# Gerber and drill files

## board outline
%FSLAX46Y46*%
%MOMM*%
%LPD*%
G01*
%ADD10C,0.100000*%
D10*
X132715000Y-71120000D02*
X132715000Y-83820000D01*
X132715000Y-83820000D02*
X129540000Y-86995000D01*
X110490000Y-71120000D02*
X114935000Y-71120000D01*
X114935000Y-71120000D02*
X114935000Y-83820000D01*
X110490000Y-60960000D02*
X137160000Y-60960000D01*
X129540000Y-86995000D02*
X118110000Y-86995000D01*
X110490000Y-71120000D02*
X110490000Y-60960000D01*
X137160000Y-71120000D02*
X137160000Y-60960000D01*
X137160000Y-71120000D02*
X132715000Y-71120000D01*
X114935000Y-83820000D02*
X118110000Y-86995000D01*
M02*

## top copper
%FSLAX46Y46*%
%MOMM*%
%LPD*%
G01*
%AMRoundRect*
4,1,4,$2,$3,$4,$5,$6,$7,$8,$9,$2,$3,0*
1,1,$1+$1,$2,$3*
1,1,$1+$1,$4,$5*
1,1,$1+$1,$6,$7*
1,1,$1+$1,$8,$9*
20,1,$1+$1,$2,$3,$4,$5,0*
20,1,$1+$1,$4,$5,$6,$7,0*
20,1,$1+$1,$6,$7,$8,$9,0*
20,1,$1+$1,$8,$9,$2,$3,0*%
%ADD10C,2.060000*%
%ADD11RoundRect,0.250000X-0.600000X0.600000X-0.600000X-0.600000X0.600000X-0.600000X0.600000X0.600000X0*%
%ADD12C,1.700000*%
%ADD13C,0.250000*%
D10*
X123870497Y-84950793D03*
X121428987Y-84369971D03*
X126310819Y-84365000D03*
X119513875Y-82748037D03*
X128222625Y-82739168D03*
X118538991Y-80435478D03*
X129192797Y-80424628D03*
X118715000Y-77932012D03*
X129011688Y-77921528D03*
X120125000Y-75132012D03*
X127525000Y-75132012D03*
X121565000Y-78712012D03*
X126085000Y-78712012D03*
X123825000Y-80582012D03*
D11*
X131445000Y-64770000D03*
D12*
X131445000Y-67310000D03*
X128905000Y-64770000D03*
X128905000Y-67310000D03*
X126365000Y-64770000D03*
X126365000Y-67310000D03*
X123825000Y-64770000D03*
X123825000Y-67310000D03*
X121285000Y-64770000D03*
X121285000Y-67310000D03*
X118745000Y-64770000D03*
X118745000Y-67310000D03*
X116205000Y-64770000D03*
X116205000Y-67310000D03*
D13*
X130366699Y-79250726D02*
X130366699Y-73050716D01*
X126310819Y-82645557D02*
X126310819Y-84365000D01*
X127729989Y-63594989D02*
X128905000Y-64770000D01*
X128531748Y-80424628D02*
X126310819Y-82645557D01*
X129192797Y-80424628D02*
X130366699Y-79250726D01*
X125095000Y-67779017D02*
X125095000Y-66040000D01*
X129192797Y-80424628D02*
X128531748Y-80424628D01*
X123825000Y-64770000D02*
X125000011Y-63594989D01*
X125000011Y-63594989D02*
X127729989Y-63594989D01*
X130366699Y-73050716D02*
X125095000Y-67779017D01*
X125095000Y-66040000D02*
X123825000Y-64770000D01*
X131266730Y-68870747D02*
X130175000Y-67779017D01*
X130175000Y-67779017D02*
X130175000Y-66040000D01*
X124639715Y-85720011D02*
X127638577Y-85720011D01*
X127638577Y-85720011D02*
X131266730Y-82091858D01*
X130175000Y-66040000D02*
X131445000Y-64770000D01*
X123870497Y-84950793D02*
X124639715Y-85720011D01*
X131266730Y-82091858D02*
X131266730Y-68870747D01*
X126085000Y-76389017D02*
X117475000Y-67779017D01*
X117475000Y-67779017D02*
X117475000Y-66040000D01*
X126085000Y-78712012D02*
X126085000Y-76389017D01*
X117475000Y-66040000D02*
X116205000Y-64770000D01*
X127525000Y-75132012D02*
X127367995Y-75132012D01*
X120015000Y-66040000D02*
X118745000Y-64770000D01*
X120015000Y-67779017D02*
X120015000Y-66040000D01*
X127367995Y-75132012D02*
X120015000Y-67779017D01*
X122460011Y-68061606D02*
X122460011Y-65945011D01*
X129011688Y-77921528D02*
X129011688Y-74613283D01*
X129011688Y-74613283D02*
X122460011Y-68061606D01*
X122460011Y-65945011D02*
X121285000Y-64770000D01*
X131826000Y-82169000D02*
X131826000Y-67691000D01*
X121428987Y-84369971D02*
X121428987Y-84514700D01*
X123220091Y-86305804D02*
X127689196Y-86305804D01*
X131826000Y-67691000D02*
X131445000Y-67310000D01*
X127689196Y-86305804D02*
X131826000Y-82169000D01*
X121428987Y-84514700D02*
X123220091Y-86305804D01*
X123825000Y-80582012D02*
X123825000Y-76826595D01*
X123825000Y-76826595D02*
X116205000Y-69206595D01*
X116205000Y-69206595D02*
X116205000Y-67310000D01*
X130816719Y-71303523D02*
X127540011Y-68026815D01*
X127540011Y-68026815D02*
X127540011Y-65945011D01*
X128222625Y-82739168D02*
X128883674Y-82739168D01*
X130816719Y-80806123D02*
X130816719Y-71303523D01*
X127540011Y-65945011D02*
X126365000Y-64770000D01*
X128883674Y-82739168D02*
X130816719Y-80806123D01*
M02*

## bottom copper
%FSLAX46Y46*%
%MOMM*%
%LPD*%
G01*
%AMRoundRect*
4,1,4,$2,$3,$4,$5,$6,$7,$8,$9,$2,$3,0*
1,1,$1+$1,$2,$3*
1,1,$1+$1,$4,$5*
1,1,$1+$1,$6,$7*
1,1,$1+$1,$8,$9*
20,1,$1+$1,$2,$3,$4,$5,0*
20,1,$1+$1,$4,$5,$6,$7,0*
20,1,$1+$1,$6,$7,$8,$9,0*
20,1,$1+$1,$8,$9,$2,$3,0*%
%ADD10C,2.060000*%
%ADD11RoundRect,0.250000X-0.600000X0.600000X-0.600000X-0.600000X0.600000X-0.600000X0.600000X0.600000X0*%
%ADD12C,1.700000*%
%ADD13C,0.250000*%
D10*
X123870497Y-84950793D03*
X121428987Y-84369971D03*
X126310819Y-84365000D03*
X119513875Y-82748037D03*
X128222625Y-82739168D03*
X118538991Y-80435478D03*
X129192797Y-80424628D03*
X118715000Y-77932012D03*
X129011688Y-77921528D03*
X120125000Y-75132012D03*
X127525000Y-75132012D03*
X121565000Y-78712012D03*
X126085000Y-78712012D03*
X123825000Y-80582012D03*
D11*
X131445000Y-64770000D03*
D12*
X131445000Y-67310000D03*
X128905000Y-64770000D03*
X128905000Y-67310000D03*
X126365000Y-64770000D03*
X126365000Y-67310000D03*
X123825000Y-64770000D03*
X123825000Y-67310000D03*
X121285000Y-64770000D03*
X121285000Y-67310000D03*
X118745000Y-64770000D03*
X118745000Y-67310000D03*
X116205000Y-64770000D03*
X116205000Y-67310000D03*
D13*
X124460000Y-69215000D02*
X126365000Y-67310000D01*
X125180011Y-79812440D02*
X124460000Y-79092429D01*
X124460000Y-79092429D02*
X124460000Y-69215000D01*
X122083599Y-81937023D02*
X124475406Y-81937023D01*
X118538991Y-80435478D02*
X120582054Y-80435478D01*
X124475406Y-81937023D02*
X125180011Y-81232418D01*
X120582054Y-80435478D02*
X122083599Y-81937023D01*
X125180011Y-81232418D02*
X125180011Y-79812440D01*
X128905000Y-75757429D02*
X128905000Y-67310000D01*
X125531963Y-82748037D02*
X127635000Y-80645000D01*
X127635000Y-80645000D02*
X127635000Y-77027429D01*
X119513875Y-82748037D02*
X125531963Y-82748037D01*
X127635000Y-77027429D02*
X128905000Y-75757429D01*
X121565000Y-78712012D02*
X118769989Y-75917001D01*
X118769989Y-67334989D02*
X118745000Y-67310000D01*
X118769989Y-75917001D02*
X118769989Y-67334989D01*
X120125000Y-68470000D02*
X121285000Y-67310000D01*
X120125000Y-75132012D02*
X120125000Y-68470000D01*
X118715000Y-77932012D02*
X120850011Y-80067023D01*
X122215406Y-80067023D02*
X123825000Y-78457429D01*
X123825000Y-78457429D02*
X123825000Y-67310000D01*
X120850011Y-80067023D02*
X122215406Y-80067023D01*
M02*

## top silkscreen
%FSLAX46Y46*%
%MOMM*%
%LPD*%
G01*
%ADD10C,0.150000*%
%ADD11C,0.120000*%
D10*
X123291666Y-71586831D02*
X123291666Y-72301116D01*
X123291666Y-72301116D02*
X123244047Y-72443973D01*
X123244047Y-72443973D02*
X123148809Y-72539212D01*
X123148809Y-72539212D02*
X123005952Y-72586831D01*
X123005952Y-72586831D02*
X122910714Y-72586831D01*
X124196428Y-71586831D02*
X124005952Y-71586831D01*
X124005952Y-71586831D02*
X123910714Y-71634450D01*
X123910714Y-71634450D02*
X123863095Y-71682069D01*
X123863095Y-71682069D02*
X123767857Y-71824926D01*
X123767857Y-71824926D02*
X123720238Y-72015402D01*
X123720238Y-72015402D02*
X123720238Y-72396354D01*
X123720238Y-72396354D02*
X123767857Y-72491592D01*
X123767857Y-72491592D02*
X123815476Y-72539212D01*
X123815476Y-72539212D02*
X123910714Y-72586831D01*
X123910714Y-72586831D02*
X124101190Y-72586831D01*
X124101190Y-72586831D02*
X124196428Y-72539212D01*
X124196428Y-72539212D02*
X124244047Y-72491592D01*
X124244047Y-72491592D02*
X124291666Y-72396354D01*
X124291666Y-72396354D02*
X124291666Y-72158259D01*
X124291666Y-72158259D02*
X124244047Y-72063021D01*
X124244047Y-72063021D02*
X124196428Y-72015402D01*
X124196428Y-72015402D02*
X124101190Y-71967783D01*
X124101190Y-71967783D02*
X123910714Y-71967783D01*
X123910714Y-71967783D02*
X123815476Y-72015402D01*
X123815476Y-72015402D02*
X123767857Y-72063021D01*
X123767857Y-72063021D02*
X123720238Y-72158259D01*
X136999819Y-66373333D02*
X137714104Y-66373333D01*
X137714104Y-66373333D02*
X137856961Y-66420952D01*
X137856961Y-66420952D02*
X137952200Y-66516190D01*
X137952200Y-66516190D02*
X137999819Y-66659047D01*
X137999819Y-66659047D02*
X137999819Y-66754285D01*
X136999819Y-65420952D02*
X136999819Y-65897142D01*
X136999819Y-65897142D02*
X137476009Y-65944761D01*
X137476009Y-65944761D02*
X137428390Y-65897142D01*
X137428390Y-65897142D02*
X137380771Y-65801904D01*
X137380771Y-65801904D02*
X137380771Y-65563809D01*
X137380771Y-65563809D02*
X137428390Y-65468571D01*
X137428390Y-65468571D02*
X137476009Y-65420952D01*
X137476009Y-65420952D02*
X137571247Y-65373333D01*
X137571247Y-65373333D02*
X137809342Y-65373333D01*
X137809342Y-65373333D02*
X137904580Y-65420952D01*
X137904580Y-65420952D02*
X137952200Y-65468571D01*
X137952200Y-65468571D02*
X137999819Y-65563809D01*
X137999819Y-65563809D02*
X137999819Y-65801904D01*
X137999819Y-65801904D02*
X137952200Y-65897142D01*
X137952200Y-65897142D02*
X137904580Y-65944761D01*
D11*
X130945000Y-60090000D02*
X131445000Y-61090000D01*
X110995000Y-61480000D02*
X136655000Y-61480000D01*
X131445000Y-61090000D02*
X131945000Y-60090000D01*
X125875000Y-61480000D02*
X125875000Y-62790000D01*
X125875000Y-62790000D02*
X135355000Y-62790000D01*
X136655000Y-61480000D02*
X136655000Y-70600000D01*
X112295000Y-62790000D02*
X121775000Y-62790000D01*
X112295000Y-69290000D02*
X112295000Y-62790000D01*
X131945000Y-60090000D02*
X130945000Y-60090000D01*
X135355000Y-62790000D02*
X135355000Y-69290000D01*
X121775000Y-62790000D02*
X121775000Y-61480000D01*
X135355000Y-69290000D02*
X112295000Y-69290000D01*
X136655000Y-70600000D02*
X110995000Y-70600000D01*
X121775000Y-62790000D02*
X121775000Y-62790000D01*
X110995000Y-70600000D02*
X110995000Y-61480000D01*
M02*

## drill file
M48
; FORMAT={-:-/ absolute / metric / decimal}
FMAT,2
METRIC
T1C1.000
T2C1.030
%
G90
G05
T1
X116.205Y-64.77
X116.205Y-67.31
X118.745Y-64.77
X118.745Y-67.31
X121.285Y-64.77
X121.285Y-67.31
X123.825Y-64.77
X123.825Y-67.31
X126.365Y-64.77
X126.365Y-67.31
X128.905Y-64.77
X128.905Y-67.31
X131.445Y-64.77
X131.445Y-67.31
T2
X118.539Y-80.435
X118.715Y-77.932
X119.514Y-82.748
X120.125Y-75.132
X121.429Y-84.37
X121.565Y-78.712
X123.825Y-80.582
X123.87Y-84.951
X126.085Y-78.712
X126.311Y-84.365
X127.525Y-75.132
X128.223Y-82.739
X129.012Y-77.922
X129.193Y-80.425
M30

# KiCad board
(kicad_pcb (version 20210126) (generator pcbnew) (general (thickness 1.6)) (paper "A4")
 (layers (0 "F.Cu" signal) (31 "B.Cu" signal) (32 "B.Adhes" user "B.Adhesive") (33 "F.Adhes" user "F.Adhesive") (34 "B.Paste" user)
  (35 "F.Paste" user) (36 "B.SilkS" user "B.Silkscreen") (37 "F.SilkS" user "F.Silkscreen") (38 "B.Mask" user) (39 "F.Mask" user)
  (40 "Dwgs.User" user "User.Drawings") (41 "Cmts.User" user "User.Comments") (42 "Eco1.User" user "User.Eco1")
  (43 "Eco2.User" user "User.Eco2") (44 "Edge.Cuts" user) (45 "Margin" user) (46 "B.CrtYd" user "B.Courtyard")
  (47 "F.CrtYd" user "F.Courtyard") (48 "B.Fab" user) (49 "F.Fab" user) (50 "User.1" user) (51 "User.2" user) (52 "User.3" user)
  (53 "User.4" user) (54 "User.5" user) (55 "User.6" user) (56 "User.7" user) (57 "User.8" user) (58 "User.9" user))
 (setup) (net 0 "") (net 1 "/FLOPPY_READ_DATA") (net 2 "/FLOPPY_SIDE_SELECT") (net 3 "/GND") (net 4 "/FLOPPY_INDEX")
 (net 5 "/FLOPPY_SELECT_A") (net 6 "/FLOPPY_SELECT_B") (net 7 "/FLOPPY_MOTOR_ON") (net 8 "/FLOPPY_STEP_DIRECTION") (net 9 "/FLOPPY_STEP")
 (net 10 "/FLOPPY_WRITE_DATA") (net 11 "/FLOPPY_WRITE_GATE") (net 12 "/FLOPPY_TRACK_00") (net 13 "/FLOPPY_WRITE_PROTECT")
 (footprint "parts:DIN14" (layer "F.Cu") (at 123.825 73.365)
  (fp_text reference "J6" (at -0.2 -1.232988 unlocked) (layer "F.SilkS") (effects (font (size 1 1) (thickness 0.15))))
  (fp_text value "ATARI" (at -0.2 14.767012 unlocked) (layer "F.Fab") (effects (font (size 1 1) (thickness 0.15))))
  (pad "1" thru_hole circle (at 0.045497 11.585793 180) (locked) (size 2.06 2.06) (drill 1.03) (layers *.Cu *.Mask)
   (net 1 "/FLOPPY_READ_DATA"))
  (pad "2" thru_hole circle (at -2.396013 11.004971 180) (locked) (size 2.06 2.06) (drill 1.03) (layers *.Cu *.Mask)
   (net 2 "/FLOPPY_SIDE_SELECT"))
  (pad "3" thru_hole circle (at 2.485819 11 180) (locked) (size 2.06 2.06) (drill 1.03) (layers *.Cu *.Mask) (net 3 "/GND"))
  (pad "4" thru_hole circle (at -4.311125 9.383037 180) (locked) (size 2.06 2.06) (drill 1.03) (layers *.Cu *.Mask) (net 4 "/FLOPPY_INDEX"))
  (pad "5" thru_hole circle (at 4.397625 9.374168 180) (locked) (size 2.06 2.06) (drill 1.03) (layers *.Cu *.Mask)
   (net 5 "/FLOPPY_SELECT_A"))
  (pad "6" thru_hole circle (at -5.286009 7.070478 180) (locked) (size 2.06 2.06) (drill 1.03) (layers *.Cu *.Mask)
   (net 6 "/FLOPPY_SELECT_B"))
  (pad "7" thru_hole circle (at 5.367797 7.059628 180) (locked) (size 2.06 2.06) (drill 1.03) (layers *.Cu *.Mask) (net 3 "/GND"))
  (pad "8" thru_hole circle (at -5.11 4.567012 180) (locked) (size 2.06 2.06) (drill 1.03) (layers *.Cu *.Mask) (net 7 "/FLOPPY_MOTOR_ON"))
  (pad "9" thru_hole circle (at 5.186688 4.556528 180) (locked) (size 2.06 2.06) (drill 1.03) (layers *.Cu *.Mask)
   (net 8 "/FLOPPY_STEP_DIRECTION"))
  (pad "10" thru_hole circle (at -3.7 1.767012 180) (locked) (size 2.06 2.06) (drill 1.03) (layers *.Cu *.Mask) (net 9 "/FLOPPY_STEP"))
  (pad "11" thru_hole circle (at 3.7 1.767012 180) (locked) (size 2.06 2.06) (drill 1.03) (layers *.Cu *.Mask) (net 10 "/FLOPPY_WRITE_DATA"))
  (pad "12" thru_hole circle (at -2.26 5.347012 180) (locked) (size 2.06 2.06) (drill 1.03) (layers *.Cu *.Mask)
   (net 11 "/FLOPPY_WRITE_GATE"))
  (pad "13" thru_hole circle (at 2.26 5.347012 180) (locked) (size 2.06 2.06) (drill 1.03) (layers *.Cu *.Mask) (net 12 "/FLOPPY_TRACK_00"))
  (pad "14" thru_hole circle (at 0 7.217012 180) (locked) (size 2.06 2.06) (drill 1.03) (layers *.Cu *.Mask)
   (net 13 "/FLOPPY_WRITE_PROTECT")))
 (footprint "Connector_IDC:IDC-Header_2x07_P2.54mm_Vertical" (layer "F.Cu") (at 131.445 64.77 -90)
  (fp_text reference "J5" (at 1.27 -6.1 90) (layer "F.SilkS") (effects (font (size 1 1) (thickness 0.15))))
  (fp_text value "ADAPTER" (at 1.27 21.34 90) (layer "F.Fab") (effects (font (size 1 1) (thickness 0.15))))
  (fp_line (start -4.68 0.5) (end -3.68 0) (layer "F.SilkS") (width 0.12))
  (fp_line (start -3.29 20.45) (end -3.29 -5.21) (layer "F.SilkS") (width 0.12))
  (fp_line (start -3.68 0) (end -4.68 -0.5) (layer "F.SilkS") (width 0.12))
  (fp_line (start -3.29 5.57) (end -1.98 5.57) (layer "F.SilkS") (width 0.12))
  (fp_line (start -1.98 5.57) (end -1.98 -3.91) (layer "F.SilkS") (width 0.12))
  (fp_line (start -3.29 -5.21) (end 5.83 -5.21) (layer "F.SilkS") (width 0.12))
  (fp_line (start -1.98 19.15) (end -1.98 9.67) (layer "F.SilkS") (width 0.12))
  (fp_line (start 4.52 19.15) (end -1.98 19.15) (layer "F.SilkS") (width 0.12))
  (fp_line (start -4.68 -0.5) (end -4.68 0.5) (layer "F.SilkS") (width 0.12))
  (fp_line (start -1.98 -3.91) (end 4.52 -3.91) (layer "F.SilkS") (width 0.12))
  (fp_line (start -1.98 9.67) (end -3.29 9.67) (layer "F.SilkS") (width 0.12))
  (fp_line (start 4.52 -3.91) (end 4.52 19.15) (layer "F.SilkS") (width 0.12))
  (fp_line (start 5.83 -5.21) (end 5.83 20.45) (layer "F.SilkS") (width 0.12))
  (fp_line (start -1.98 9.67) (end -1.98 9.67) (layer "F.SilkS") (width 0.12))
  (fp_line (start 5.83 20.45) (end -3.29 20.45) (layer "F.SilkS") (width 0.12))
  (pad "1" thru_hole roundrect (at 0 0 270) (locked) (size 1.7 1.7) (drill 1) (layers *.Cu *.Mask) (roundrect_rratio 0.1470588235294118)
   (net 1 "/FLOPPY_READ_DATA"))
  (pad "2" thru_hole circle (at 2.54 0 270) (locked) (size 1.7 1.7) (drill 1) (layers *.Cu *.Mask) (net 2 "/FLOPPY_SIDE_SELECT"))
  (pad "3" thru_hole circle (at 0 2.54 270) (locked) (size 1.7 1.7) (drill 1) (layers *.Cu *.Mask) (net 3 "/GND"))
  (pad "4" thru_hole circle (at 2.54 2.54 270) (locked) (size 1.7 1.7) (drill 1) (layers *.Cu *.Mask) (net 4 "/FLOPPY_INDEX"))
  (pad "5" thru_hole circle (at 0 5.08 270) (locked) (size 1.7 1.7) (drill 1) (layers *.Cu *.Mask) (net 5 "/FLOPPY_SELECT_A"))
  (pad "6" thru_hole circle (at 2.54 5.08 270) (locked) (size 1.7 1.7) (drill 1) (layers *.Cu *.Mask) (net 6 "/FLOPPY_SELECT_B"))
  (pad "7" thru_hole circle (at 0 7.62 270) (locked) (size 1.7 1.7) (drill 1) (layers *.Cu *.Mask) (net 3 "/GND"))
  (pad "8" thru_hole circle (at 2.54 7.62 270) (locked) (size 1.7 1.7) (drill 1) (layers *.Cu *.Mask) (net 7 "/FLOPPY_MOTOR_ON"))
  (pad "9" thru_hole circle (at 0 10.16 270) (locked) (size 1.7 1.7) (drill 1) (layers *.Cu *.Mask) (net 8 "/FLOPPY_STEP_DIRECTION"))
  (pad "10" thru_hole circle (at 2.54 10.16 270) (locked) (size 1.7 1.7) (drill 1) (layers *.Cu *.Mask) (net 9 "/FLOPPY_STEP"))
  (pad "11" thru_hole circle (at 0 12.7 270) (locked) (size 1.7 1.7) (drill 1) (layers *.Cu *.Mask) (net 10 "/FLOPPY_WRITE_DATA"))
  (pad "12" thru_hole circle (at 2.54 12.7 270) (locked) (size 1.7 1.7) (drill 1) (layers *.Cu *.Mask) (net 11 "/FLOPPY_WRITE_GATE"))
  (pad "13" thru_hole circle (at 0 15.24 270) (locked) (size 1.7 1.7) (drill 1) (layers *.Cu *.Mask) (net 12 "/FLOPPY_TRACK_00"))
  (pad "14" thru_hole circle (at 2.54 15.24 270) (locked) (size 1.7 1.7) (drill 1) (layers *.Cu *.Mask) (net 13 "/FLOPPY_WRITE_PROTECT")))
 (gr_line (start 132.715 71.12) (end 132.715 83.82) (layer "Edge.Cuts") (width 0.1))
 (gr_line (start 132.715 83.82) (end 129.54 86.995) (layer "Edge.Cuts") (width 0.1))
 (gr_line (start 110.49 71.12) (end 114.935 71.12) (layer "Edge.Cuts") (width 0.1))
 (gr_line (start 114.935 71.12) (end 114.935 83.82) (layer "Edge.Cuts") (width 0.1))
 (gr_line (start 110.49 60.96) (end 137.16 60.96) (layer "Edge.Cuts") (width 0.1))
 (gr_line (start 129.54 86.995) (end 118.11 86.995) (layer "Edge.Cuts") (width 0.1))
 (gr_line (start 110.49 71.12) (end 110.49 60.96) (layer "Edge.Cuts") (width 0.1))
 (gr_line (start 137.16 71.12) (end 137.16 60.96) (layer "Edge.Cuts") (width 0.1))
 (gr_line (start 137.16 71.12) (end 132.715 71.12) (layer "Edge.Cuts") (width 0.1))
 (gr_line (start 114.935 83.82) (end 118.11 86.995) (layer "Edge.Cuts") (width 0.1))
 (segment (start 130.366699 79.250726) (end 130.366699 73.050716) (width 0.25) (layer "F.Cu") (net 3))
 (segment (start 126.310819 82.645557) (end 126.310819 84.365) (width 0.25) (layer "F.Cu") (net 3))
 (segment (start 127.729989 63.594989) (end 128.905 64.77) (width 0.25) (layer "F.Cu") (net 3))
 (segment (start 128.531748 80.424628) (end 126.310819 82.645557) (width 0.25) (layer "F.Cu") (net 3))
 (segment (start 129.192797 80.424628) (end 130.366699 79.250726) (width 0.25) (layer "F.Cu") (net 3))
 (segment (start 125.095 67.779017) (end 125.095 66.04) (width 0.25) (layer "F.Cu") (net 3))
 (segment (start 129.192797 80.424628) (end 128.531748 80.424628) (width 0.25) (layer "F.Cu") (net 3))
 (segment (start 123.825 64.77) (end 125.000011 63.594989) (width 0.25) (layer "F.Cu") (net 3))
 (segment (start 125.000011 63.594989) (end 127.729989 63.594989) (width 0.25) (layer "F.Cu") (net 3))
 (segment (start 130.366699 73.050716) (end 125.095 67.779017) (width 0.25) (layer "F.Cu") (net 3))
 (segment (start 125.095 66.04) (end 123.825 64.77) (width 0.25) (layer "F.Cu") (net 3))
 (segment (start 131.26673 68.870747) (end 130.175 67.779017) (width 0.25) (layer "F.Cu") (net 1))
 (segment (start 130.175 67.779017) (end 130.175 66.04) (width 0.25) (layer "F.Cu") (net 1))
 (segment (start 124.639715 85.720011) (end 127.638577 85.720011) (width 0.25) (layer "F.Cu") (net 1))
 (segment (start 127.638577 85.720011) (end 131.26673 82.091858) (width 0.25) (layer "F.Cu") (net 1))
 (segment (start 130.175 66.04) (end 131.445 64.77) (width 0.25) (layer "F.Cu") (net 1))
 (segment (start 123.870497 84.950793) (end 124.639715 85.720011) (width 0.25) (layer "F.Cu") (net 1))
 (segment (start 131.26673 82.091858) (end 131.26673 68.870747) (width 0.25) (layer "F.Cu") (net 1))
 (segment (start 126.085 76.389017) (end 117.475 67.779017) (width 0.25) (layer "F.Cu") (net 12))
 (segment (start 117.475 67.779017) (end 117.475 66.04) (width 0.25) (layer "F.Cu") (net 12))
 (segment (start 126.085 78.712012) (end 126.085 76.389017) (width 0.25) (layer "F.Cu") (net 12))
 (segment (start 117.475 66.04) (end 116.205 64.77) (width 0.25) (layer "F.Cu") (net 12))
 (segment (start 127.525 75.132012) (end 127.367995 75.132012) (width 0.25) (layer "F.Cu") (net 10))
 (segment (start 120.015 66.04) (end 118.745 64.77) (width 0.25) (layer "F.Cu") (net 10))
 (segment (start 120.015 67.779017) (end 120.015 66.04) (width 0.25) (layer "F.Cu") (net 10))
 (segment (start 127.367995 75.132012) (end 120.015 67.779017) (width 0.25) (layer "F.Cu") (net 10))
 (segment (start 122.460011 68.061606) (end 122.460011 65.945011) (width 0.25) (layer "F.Cu") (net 8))
 (segment (start 129.011688 77.921528) (end 129.011688 74.613283) (width 0.25) (layer "F.Cu") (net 8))
 (segment (start 129.011688 74.613283) (end 122.460011 68.061606) (width 0.25) (layer "F.Cu") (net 8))
 (segment (start 122.460011 65.945011) (end 121.285 64.77) (width 0.25) (layer "F.Cu") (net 8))
 (segment (start 124.46 69.215) (end 126.365 67.31) (width 0.25) (layer "B.Cu") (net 6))
 (segment (start 125.180011 79.81244) (end 124.46 79.092429) (width 0.25) (layer "B.Cu") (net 6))
 (segment (start 124.46 79.092429) (end 124.46 69.215) (width 0.25) (layer "B.Cu") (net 6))
 (segment (start 122.083599 81.937023) (end 124.475406 81.937023) (width 0.25) (layer "B.Cu") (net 6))
 (segment (start 118.538991 80.435478) (end 120.582054 80.435478) (width 0.25) (layer "B.Cu") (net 6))
 (segment (start 124.475406 81.937023) (end 125.180011 81.232418) (width 0.25) (layer "B.Cu") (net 6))
 (segment (start 120.582054 80.435478) (end 122.083599 81.937023) (width 0.25) (layer "B.Cu") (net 6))
 (segment (start 125.180011 81.232418) (end 125.180011 79.81244) (width 0.25) (layer "B.Cu") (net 6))
 (segment (start 128.905 75.757429) (end 128.905 67.31) (width 0.25) (layer "B.Cu") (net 4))
 (segment (start 125.531963 82.748037) (end 127.635 80.645) (width 0.25) (layer "B.Cu") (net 4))
 (segment (start 127.635 80.645) (end 127.635 77.027429) (width 0.25) (layer "B.Cu") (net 4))
 (segment (start 119.513875 82.748037) (end 125.531963 82.748037) (width 0.25) (layer "B.Cu") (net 4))
 (segment (start 127.635 77.027429) (end 128.905 75.757429) (width 0.25) (layer "B.Cu") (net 4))
 (segment (start 131.826 82.169) (end 131.826 67.691) (width 0.25) (layer "F.Cu") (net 2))
 (segment (start 121.428987 84.369971) (end 121.428987 84.5147) (width 0.25) (layer "F.Cu") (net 2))
 (segment (start 123.220091 86.305804) (end 127.689196 86.305804) (width 0.25) (layer "F.Cu") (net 2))
 (segment (start 131.826 67.691) (end 131.445 67.31) (width 0.25) (layer "F.Cu") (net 2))
 (segment (start 127.689196 86.305804) (end 131.826 82.169) (width 0.25) (layer "F.Cu") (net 2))
 (segment (start 121.428987 84.5147) (end 123.220091 86.305804) (width 0.25) (layer "F.Cu") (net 2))
 (segment (start 123.825 80.582012) (end 123.825 76.826595) (width 0.25) (layer "F.Cu") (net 13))
 (segment (start 123.825 76.826595) (end 116.205 69.206595) (width 0.25) (layer "F.Cu") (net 13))
 (segment (start 116.205 69.206595) (end 116.205 67.31) (width 0.25) (layer "F.Cu") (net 13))
 (segment (start 121.565 78.712012) (end 118.769989 75.917001) (width 0.25) (layer "B.Cu") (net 11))
 (segment (start 118.769989 67.334989) (end 118.745 67.31) (width 0.25) (layer "B.Cu") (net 11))
 (segment (start 118.769989 75.917001) (end 118.769989 67.334989) (width 0.25) (layer "B.Cu") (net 11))
 (segment (start 120.125 68.47) (end 121.285 67.31) (width 0.25) (layer "B.Cu") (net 9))
 (segment (start 120.125 75.132012) (end 120.125 68.47) (width 0.25) (layer "B.Cu") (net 9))
 (segment (start 118.715 77.932012) (end 120.850011 80.067023) (width 0.25) (layer "B.Cu") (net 7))
 (segment (start 122.215406 80.067023) (end 123.825 78.457429) (width 0.25) (layer "B.Cu") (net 7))
 (segment (start 123.825 78.457429) (end 123.825 67.31) (width 0.25) (layer "B.Cu") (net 7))
 (segment (start 120.850011 80.067023) (end 122.215406 80.067023) (width 0.25) (layer "B.Cu") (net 7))
 (segment (start 130.816719 71.303523) (end 127.540011 68.026815) (width 0.25) (layer "F.Cu") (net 5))
 (segment (start 127.540011 68.026815) (end 127.540011 65.945011) (width 0.25) (layer "F.Cu") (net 5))
 (segment (start 128.222625 82.739168) (end 128.883674 82.739168) (width 0.25) (layer "F.Cu") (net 5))
 (segment (start 130.816719 80.806123) (end 130.816719 71.303523) (width 0.25) (layer "F.Cu") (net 5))
 (segment (start 127.540011 65.945011) (end 126.365 64.77) (width 0.25) (layer "F.Cu") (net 5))
 (segment (start 128.883674 82.739168) (end 130.816719 80.806123) (width 0.25) (layer "F.Cu") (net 5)))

